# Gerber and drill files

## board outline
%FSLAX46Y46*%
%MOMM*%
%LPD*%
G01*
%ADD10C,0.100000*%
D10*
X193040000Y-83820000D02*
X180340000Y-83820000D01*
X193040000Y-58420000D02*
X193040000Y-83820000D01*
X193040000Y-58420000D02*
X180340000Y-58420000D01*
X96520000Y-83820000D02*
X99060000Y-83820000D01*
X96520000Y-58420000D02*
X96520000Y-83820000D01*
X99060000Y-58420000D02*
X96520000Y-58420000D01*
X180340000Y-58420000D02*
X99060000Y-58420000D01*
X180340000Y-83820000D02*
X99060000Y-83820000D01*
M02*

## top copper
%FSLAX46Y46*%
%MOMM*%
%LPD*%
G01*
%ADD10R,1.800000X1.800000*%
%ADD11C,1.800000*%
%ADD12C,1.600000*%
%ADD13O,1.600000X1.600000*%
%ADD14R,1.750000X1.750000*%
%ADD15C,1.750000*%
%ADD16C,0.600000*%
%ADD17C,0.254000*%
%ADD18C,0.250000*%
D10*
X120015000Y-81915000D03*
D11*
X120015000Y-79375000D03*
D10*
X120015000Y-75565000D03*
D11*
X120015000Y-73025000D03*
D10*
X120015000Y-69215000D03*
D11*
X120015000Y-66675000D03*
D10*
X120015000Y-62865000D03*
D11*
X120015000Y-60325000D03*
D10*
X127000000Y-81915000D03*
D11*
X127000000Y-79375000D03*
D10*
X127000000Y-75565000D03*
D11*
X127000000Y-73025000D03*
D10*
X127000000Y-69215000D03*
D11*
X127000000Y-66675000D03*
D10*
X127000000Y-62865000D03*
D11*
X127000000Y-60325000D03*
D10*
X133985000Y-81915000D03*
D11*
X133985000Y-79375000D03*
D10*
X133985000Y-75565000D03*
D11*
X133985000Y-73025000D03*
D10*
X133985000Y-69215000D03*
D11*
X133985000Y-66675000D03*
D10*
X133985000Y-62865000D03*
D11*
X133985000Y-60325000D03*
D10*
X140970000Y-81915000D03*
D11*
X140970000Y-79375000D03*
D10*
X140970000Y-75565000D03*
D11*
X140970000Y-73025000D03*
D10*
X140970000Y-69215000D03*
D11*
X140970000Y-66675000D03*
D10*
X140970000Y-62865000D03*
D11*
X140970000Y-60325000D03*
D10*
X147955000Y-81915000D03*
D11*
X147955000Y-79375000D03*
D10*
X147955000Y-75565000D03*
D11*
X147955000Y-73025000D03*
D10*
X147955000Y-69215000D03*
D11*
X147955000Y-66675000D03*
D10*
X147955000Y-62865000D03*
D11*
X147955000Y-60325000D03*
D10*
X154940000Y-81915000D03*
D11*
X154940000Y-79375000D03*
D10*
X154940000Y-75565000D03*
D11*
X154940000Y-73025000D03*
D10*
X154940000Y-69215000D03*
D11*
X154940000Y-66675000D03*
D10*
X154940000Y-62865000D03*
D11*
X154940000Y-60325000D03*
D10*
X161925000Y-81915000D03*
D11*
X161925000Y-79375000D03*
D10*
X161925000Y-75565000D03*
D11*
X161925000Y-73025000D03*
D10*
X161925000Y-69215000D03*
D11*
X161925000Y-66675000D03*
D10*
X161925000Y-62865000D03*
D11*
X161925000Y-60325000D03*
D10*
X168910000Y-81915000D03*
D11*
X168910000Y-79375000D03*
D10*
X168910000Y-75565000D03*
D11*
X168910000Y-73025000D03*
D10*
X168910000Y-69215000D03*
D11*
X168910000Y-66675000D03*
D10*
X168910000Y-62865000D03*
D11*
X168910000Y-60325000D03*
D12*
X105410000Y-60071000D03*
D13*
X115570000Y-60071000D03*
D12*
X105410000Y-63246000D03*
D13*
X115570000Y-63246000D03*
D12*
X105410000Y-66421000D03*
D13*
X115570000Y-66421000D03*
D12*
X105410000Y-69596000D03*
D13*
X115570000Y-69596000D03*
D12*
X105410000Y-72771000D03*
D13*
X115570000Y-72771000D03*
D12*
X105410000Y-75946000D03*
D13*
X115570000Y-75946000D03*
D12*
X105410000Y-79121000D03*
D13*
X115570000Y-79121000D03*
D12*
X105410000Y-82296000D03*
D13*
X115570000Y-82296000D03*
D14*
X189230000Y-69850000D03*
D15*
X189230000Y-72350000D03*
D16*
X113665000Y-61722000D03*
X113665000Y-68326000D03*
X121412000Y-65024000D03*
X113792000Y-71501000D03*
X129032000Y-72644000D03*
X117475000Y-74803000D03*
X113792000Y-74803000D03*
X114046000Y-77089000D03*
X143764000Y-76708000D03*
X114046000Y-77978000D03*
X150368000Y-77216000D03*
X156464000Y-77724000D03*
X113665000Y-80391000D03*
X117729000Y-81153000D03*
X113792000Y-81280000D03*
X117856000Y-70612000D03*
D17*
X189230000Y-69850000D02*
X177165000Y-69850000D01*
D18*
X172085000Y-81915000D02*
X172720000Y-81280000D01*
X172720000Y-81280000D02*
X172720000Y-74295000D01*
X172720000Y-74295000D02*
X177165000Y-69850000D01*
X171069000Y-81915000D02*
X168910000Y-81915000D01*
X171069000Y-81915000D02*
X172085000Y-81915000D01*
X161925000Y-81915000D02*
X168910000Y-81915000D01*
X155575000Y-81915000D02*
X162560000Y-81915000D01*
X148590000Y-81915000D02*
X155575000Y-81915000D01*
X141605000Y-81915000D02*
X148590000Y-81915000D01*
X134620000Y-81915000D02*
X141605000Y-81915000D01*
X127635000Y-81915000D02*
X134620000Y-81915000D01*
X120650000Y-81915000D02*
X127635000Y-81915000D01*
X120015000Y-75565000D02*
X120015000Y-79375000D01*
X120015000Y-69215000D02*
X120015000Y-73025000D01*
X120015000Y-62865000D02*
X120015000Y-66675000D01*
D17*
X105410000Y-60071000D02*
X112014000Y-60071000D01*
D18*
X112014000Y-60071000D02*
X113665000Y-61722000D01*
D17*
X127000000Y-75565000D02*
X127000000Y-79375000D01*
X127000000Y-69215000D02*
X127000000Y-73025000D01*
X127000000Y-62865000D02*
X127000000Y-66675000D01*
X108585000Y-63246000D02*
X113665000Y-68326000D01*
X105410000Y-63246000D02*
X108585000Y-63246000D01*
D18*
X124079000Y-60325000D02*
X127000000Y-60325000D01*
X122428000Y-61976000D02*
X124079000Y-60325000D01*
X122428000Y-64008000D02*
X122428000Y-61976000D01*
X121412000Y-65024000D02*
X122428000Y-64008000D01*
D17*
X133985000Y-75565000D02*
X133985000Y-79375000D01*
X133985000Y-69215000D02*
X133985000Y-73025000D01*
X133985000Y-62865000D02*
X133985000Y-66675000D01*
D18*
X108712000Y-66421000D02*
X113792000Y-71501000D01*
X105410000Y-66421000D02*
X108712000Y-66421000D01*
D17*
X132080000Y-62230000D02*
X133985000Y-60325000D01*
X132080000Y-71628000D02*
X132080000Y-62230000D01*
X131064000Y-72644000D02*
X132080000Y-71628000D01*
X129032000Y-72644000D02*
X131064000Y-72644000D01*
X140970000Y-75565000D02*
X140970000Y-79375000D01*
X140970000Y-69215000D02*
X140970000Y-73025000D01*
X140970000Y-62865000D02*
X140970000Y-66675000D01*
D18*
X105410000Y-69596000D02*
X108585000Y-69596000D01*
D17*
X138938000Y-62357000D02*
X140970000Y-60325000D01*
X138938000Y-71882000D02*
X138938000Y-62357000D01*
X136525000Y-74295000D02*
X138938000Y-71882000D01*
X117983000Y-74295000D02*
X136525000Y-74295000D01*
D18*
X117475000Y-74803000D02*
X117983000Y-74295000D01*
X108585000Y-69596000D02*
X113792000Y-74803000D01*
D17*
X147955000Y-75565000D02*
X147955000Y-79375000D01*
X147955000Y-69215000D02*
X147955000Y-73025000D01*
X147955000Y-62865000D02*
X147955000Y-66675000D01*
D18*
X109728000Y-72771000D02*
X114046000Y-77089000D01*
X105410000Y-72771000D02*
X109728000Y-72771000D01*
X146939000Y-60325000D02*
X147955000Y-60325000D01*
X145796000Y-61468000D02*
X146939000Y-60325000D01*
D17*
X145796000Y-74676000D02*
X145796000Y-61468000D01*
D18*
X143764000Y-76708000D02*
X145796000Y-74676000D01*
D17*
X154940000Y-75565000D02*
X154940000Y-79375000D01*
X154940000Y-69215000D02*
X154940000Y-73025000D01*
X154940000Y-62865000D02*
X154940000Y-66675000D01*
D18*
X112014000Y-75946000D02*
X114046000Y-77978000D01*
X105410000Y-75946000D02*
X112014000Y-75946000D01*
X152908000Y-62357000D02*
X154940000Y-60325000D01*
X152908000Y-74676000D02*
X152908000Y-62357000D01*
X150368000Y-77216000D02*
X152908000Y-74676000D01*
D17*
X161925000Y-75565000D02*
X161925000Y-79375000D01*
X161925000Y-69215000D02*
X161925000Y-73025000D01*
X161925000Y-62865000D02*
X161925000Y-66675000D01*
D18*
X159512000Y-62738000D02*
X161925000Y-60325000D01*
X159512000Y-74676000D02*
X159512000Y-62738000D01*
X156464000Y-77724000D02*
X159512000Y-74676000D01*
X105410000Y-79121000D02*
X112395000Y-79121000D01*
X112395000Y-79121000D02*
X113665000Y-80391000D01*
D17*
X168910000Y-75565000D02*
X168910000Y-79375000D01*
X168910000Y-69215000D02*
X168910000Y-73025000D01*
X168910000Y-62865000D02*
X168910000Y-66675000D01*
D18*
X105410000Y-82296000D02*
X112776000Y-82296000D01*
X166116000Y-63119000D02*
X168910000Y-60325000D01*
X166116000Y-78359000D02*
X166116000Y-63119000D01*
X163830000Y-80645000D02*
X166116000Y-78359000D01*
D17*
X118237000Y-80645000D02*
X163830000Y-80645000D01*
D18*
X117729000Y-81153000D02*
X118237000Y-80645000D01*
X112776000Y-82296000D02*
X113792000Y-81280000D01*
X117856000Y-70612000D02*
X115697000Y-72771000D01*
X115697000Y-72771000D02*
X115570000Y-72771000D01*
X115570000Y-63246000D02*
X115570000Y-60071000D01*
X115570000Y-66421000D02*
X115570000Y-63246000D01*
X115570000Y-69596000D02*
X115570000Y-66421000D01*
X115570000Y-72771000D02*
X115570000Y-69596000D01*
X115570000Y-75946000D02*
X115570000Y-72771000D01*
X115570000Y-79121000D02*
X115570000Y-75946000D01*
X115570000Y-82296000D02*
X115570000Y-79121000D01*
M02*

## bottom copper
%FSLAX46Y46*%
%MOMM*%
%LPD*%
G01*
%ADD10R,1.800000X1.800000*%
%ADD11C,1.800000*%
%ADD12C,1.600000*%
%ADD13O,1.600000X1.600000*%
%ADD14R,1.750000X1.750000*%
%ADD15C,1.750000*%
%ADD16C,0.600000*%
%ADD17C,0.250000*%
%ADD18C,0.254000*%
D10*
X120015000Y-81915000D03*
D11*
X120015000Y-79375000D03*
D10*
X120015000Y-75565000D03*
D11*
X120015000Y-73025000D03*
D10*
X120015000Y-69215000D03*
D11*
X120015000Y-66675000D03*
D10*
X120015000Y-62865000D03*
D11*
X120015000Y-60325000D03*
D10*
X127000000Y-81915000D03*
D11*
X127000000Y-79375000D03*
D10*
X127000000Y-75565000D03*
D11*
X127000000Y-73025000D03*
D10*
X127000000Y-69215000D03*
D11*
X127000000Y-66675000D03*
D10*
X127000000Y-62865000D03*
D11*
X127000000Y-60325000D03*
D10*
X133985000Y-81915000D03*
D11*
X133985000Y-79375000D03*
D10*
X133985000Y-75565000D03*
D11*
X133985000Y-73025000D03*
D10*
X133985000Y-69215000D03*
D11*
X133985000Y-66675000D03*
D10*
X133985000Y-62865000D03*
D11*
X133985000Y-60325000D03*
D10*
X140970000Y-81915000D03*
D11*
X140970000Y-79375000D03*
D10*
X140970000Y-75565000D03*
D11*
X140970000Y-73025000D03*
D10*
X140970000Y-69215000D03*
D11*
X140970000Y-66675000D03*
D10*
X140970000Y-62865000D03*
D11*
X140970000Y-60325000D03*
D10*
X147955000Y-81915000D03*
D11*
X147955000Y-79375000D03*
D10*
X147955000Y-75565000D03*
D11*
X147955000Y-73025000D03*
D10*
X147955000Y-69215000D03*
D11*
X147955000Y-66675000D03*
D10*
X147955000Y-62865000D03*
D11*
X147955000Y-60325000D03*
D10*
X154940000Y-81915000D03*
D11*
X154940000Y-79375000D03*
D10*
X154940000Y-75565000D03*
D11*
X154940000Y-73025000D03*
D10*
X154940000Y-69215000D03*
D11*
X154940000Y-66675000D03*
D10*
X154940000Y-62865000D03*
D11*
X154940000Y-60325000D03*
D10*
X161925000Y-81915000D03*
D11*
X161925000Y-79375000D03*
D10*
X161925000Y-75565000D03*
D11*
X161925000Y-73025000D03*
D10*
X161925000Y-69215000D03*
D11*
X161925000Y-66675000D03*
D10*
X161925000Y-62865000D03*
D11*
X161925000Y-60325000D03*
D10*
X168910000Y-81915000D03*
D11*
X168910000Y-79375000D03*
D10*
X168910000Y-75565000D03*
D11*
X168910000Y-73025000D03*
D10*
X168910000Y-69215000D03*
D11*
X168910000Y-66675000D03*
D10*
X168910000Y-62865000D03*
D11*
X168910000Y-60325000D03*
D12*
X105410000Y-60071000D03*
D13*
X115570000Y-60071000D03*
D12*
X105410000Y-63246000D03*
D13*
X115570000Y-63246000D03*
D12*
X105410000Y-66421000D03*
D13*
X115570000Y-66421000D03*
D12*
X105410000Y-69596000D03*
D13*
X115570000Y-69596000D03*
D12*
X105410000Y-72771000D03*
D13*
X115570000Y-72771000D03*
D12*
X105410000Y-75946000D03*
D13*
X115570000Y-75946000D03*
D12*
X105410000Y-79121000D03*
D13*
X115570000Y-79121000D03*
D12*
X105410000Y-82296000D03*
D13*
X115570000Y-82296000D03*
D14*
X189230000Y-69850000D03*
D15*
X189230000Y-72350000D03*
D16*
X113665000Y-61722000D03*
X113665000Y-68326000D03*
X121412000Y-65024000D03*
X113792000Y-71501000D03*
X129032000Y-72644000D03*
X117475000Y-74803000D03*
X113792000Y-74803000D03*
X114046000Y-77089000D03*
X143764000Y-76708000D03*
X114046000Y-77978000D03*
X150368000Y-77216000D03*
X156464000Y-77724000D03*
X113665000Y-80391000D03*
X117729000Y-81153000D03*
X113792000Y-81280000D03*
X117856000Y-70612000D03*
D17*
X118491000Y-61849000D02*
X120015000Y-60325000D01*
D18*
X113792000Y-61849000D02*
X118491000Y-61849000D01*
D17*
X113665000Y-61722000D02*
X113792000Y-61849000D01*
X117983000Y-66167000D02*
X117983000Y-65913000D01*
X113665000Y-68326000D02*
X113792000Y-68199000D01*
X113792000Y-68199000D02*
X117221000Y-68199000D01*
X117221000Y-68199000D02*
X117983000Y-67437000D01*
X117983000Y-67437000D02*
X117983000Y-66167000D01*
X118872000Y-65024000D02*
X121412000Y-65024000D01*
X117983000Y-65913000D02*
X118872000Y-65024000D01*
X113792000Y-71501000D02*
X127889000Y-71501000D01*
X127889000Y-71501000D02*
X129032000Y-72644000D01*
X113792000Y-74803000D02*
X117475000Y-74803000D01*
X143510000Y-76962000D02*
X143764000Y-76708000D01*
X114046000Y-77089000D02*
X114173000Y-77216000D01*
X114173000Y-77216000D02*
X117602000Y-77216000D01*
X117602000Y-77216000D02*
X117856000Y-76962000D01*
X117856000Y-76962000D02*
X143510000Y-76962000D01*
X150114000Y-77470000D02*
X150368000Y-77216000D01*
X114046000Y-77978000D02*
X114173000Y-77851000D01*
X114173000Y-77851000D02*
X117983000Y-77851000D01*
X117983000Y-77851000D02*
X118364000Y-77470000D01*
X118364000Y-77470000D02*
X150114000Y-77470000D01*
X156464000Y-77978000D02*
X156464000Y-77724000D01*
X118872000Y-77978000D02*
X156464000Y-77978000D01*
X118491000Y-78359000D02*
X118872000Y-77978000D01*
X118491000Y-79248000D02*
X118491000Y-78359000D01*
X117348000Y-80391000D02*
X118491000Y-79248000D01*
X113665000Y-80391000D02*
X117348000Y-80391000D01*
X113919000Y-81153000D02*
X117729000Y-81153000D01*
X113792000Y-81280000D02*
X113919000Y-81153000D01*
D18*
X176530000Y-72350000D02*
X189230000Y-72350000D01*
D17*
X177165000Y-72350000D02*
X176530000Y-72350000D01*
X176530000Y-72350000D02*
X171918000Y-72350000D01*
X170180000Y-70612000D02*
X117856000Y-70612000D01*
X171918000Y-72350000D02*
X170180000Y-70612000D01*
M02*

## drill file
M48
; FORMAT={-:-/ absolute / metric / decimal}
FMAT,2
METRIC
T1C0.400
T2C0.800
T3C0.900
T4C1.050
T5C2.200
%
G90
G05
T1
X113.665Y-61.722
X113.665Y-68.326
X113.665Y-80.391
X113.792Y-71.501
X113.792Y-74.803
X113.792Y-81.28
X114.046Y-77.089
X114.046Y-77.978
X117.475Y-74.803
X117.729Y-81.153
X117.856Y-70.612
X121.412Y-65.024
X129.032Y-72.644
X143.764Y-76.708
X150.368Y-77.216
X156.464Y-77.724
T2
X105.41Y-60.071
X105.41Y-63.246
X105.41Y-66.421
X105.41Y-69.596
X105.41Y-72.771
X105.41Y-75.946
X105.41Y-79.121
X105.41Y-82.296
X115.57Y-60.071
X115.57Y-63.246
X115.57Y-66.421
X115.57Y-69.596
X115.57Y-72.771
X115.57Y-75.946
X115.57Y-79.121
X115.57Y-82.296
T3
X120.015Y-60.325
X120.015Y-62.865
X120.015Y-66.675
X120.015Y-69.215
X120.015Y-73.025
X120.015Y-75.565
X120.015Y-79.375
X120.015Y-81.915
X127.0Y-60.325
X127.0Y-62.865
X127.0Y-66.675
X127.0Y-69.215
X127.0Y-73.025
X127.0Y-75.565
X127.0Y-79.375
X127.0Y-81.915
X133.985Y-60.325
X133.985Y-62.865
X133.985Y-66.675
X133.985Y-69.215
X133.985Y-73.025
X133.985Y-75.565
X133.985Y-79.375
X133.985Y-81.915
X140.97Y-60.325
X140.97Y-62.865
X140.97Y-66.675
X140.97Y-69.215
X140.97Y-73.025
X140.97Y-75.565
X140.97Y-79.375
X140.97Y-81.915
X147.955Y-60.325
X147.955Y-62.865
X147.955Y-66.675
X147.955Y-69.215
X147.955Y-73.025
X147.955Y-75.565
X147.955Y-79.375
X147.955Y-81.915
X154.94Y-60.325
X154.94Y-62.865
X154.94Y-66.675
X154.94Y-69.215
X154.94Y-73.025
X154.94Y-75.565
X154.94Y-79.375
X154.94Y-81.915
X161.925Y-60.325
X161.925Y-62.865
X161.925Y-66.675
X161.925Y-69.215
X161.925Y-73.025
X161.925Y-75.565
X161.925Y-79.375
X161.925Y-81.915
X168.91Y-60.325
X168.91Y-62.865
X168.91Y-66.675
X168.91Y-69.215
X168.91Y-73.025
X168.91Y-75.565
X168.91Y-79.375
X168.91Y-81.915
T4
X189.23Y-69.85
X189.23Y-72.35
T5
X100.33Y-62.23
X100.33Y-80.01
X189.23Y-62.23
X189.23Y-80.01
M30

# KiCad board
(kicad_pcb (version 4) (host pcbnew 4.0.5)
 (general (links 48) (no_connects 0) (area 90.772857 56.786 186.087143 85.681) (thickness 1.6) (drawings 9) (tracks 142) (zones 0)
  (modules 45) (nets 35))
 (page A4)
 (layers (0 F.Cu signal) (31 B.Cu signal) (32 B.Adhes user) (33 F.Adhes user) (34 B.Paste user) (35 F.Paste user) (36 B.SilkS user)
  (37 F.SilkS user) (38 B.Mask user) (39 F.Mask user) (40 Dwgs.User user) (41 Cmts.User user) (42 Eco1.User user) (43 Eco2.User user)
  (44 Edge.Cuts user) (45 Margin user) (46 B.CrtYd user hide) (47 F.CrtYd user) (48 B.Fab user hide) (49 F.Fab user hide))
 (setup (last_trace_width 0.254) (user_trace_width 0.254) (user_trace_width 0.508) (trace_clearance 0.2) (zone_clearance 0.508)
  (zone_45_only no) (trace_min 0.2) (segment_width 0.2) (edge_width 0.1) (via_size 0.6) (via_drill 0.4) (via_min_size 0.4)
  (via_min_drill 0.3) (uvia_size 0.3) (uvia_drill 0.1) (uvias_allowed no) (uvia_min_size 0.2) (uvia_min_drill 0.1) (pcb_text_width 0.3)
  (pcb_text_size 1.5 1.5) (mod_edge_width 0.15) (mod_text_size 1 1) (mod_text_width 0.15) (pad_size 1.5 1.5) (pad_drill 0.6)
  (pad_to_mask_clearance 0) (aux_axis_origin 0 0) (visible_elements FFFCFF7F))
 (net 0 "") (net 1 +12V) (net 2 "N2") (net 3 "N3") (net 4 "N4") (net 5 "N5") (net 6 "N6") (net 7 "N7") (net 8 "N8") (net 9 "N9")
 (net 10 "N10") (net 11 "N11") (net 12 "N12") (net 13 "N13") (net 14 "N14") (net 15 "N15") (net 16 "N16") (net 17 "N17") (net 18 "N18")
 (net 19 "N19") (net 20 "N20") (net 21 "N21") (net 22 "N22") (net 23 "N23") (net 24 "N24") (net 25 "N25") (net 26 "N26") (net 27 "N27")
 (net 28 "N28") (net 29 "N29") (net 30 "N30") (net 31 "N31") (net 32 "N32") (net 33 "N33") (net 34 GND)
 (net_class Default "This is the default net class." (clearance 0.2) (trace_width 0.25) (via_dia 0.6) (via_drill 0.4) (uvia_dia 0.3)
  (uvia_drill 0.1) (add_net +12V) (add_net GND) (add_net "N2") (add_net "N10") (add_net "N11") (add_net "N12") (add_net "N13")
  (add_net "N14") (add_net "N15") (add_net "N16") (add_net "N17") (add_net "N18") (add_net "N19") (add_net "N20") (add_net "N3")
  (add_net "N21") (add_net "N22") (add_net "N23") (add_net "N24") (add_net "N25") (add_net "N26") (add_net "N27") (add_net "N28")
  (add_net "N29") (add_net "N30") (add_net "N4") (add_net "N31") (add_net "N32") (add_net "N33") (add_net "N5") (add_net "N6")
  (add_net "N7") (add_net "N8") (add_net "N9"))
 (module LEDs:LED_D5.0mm (layer F.Cu) (at 120.015 81.915 90)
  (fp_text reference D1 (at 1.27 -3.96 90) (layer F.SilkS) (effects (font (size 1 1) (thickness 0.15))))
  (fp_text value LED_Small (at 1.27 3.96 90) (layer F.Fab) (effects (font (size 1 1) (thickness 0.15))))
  (pad 1 thru_hole rect (at 0 0 90) (size 1.8 1.8) (drill 0.9) (layers *.Cu *.Mask) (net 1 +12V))
  (pad 2 thru_hole circle (at 2.54 0 90) (size 1.8 1.8) (drill 0.9) (layers *.Cu *.Mask) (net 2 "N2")))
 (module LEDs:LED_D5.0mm (layer F.Cu) (at 120.015 75.565 90)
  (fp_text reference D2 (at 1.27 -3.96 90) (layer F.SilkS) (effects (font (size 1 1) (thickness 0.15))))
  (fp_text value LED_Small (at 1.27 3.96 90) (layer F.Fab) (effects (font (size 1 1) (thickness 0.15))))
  (pad 1 thru_hole rect (at 0 0 90) (size 1.8 1.8) (drill 0.9) (layers *.Cu *.Mask) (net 2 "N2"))
  (pad 2 thru_hole circle (at 2.54 0 90) (size 1.8 1.8) (drill 0.9) (layers *.Cu *.Mask) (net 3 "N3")))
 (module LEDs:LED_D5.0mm (layer F.Cu) (at 120.015 69.215 90)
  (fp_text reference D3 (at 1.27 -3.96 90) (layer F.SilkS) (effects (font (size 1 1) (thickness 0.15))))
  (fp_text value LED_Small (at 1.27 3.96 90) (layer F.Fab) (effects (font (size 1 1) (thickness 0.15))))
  (pad 1 thru_hole rect (at 0 0 90) (size 1.8 1.8) (drill 0.9) (layers *.Cu *.Mask) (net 3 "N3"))
  (pad 2 thru_hole circle (at 2.54 0 90) (size 1.8 1.8) (drill 0.9) (layers *.Cu *.Mask) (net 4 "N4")))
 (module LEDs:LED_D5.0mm (layer F.Cu) (at 120.015 62.865 90)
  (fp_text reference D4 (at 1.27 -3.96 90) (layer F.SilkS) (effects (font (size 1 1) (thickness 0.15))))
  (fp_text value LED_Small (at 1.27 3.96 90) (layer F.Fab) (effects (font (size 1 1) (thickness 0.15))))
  (pad 1 thru_hole rect (at 0 0 90) (size 1.8 1.8) (drill 0.9) (layers *.Cu *.Mask) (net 4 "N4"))
  (pad 2 thru_hole circle (at 2.54 0 90) (size 1.8 1.8) (drill 0.9) (layers *.Cu *.Mask) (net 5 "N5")))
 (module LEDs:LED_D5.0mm (layer F.Cu) (at 127 81.915 90)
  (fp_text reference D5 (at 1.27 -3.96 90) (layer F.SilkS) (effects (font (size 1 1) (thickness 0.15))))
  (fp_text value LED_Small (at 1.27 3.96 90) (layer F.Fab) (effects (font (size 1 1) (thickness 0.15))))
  (pad 1 thru_hole rect (at 0 0 90) (size 1.8 1.8) (drill 0.9) (layers *.Cu *.Mask) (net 1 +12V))
  (pad 2 thru_hole circle (at 2.54 0 90) (size 1.8 1.8) (drill 0.9) (layers *.Cu *.Mask) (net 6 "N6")))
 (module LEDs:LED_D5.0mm (layer F.Cu) (at 127 75.565 90)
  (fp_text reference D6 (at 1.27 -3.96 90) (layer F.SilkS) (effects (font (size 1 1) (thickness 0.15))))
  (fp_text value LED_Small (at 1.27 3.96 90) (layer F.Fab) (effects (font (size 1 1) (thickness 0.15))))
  (pad 1 thru_hole rect (at 0 0 90) (size 1.8 1.8) (drill 0.9) (layers *.Cu *.Mask) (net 6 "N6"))
  (pad 2 thru_hole circle (at 2.54 0 90) (size 1.8 1.8) (drill 0.9) (layers *.Cu *.Mask) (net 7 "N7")))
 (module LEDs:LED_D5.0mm (layer F.Cu) (at 127 69.215 90)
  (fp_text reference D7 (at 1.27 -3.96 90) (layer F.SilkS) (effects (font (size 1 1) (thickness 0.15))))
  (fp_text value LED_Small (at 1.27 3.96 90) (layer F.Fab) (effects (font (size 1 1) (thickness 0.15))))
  (pad 1 thru_hole rect (at 0 0 90) (size 1.8 1.8) (drill 0.9) (layers *.Cu *.Mask) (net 7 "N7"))
  (pad 2 thru_hole circle (at 2.54 0 90) (size 1.8 1.8) (drill 0.9) (layers *.Cu *.Mask) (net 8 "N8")))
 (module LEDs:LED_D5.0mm (layer F.Cu) (at 127 62.865 90)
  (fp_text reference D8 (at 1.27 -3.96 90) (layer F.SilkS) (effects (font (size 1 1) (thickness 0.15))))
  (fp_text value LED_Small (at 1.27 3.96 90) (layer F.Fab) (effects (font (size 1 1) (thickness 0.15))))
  (pad 1 thru_hole rect (at 0 0 90) (size 1.8 1.8) (drill 0.9) (layers *.Cu *.Mask) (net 8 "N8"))
  (pad 2 thru_hole circle (at 2.54 0 90) (size 1.8 1.8) (drill 0.9) (layers *.Cu *.Mask) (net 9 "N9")))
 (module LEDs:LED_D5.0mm (layer F.Cu) (at 133.985 81.915 90)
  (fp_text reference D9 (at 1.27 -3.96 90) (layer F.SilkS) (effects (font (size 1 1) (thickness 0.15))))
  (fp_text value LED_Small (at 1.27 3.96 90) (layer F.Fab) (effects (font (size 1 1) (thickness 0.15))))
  (pad 1 thru_hole rect (at 0 0 90) (size 1.8 1.8) (drill 0.9) (layers *.Cu *.Mask) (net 1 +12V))
  (pad 2 thru_hole circle (at 2.54 0 90) (size 1.8 1.8) (drill 0.9) (layers *.Cu *.Mask) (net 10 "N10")))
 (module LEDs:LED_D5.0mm (layer F.Cu) (at 133.985 75.565 90)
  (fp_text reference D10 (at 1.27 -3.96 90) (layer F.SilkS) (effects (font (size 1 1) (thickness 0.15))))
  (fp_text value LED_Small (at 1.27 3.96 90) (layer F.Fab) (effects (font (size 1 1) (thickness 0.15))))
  (pad 1 thru_hole rect (at 0 0 90) (size 1.8 1.8) (drill 0.9) (layers *.Cu *.Mask) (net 10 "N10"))
  (pad 2 thru_hole circle (at 2.54 0 90) (size 1.8 1.8) (drill 0.9) (layers *.Cu *.Mask) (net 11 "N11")))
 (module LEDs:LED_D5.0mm (layer F.Cu) (at 133.985 69.215 90)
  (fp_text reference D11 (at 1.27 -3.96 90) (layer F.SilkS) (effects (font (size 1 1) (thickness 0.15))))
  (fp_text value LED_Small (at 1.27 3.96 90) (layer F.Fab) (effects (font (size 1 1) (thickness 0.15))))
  (pad 1 thru_hole rect (at 0 0 90) (size 1.8 1.8) (drill 0.9) (layers *.Cu *.Mask) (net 11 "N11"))
  (pad 2 thru_hole circle (at 2.54 0 90) (size 1.8 1.8) (drill 0.9) (layers *.Cu *.Mask) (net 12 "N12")))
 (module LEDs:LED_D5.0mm (layer F.Cu) (at 133.985 62.865 90)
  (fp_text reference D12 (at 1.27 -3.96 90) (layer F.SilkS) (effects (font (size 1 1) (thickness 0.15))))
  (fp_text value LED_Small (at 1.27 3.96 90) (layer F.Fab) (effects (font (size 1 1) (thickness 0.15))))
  (pad 1 thru_hole rect (at 0 0 90) (size 1.8 1.8) (drill 0.9) (layers *.Cu *.Mask) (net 12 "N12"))
  (pad 2 thru_hole circle (at 2.54 0 90) (size 1.8 1.8) (drill 0.9) (layers *.Cu *.Mask) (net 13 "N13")))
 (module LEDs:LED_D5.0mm (layer F.Cu) (at 140.97 81.915 90)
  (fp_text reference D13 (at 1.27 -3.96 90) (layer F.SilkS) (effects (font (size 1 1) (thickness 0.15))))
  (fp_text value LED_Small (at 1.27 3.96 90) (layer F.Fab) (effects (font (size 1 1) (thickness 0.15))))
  (pad 1 thru_hole rect (at 0 0 90) (size 1.8 1.8) (drill 0.9) (layers *.Cu *.Mask) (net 1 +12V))
  (pad 2 thru_hole circle (at 2.54 0 90) (size 1.8 1.8) (drill 0.9) (layers *.Cu *.Mask) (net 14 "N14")))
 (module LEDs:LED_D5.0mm (layer F.Cu) (at 140.97 75.565 90)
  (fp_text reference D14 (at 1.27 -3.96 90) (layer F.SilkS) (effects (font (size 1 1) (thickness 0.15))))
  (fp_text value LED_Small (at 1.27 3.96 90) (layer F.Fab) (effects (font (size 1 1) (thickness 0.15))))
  (pad 1 thru_hole rect (at 0 0 90) (size 1.8 1.8) (drill 0.9) (layers *.Cu *.Mask) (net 14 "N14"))
  (pad 2 thru_hole circle (at 2.54 0 90) (size 1.8 1.8) (drill 0.9) (layers *.Cu *.Mask) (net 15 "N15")))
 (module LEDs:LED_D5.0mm (layer F.Cu) (at 140.97 69.215 90)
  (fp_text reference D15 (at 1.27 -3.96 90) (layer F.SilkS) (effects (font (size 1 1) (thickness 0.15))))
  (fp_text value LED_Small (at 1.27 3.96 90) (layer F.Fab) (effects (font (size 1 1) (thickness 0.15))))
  (pad 1 thru_hole rect (at 0 0 90) (size 1.8 1.8) (drill 0.9) (layers *.Cu *.Mask) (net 15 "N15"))
  (pad 2 thru_hole circle (at 2.54 0 90) (size 1.8 1.8) (drill 0.9) (layers *.Cu *.Mask) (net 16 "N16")))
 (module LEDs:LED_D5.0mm (layer F.Cu) (at 140.97 62.865 90)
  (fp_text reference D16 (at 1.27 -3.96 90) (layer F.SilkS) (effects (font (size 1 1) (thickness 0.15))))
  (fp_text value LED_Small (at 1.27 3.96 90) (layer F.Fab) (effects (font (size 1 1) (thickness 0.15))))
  (pad 1 thru_hole rect (at 0 0 90) (size 1.8 1.8) (drill 0.9) (layers *.Cu *.Mask) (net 16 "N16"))
  (pad 2 thru_hole circle (at 2.54 0 90) (size 1.8 1.8) (drill 0.9) (layers *.Cu *.Mask) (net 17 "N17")))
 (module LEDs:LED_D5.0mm (layer F.Cu) (at 147.955 81.915 90)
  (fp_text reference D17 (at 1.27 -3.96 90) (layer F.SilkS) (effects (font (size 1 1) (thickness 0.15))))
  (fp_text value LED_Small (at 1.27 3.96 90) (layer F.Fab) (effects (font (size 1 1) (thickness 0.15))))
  (pad 1 thru_hole rect (at 0 0 90) (size 1.8 1.8) (drill 0.9) (layers *.Cu *.Mask) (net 1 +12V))
  (pad 2 thru_hole circle (at 2.54 0 90) (size 1.8 1.8) (drill 0.9) (layers *.Cu *.Mask) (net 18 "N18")))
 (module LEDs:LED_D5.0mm (layer F.Cu) (at 147.955 75.565 90)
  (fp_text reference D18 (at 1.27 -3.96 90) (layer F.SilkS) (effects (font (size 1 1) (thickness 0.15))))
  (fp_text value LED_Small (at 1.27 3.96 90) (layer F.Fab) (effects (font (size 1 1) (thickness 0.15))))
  (pad 1 thru_hole rect (at 0 0 90) (size 1.8 1.8) (drill 0.9) (layers *.Cu *.Mask) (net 18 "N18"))
  (pad 2 thru_hole circle (at 2.54 0 90) (size 1.8 1.8) (drill 0.9) (layers *.Cu *.Mask) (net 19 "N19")))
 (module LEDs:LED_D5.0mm (layer F.Cu) (at 147.955 69.215 90)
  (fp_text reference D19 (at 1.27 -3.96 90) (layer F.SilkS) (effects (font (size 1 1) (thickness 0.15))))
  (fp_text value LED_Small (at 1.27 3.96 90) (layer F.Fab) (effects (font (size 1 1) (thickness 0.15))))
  (pad 1 thru_hole rect (at 0 0 90) (size 1.8 1.8) (drill 0.9) (layers *.Cu *.Mask) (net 19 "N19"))
  (pad 2 thru_hole circle (at 2.54 0 90) (size 1.8 1.8) (drill 0.9) (layers *.Cu *.Mask) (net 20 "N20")))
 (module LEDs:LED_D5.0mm (layer F.Cu) (at 147.955 62.865 90)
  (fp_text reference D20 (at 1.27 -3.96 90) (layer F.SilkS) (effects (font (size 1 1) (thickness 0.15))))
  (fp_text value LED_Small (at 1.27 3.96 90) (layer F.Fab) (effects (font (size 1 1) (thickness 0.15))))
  (pad 1 thru_hole rect (at 0 0 90) (size 1.8 1.8) (drill 0.9) (layers *.Cu *.Mask) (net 20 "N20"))
  (pad 2 thru_hole circle (at 2.54 0 90) (size 1.8 1.8) (drill 0.9) (layers *.Cu *.Mask) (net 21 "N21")))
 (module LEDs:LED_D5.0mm (layer F.Cu) (at 154.94 81.915 90)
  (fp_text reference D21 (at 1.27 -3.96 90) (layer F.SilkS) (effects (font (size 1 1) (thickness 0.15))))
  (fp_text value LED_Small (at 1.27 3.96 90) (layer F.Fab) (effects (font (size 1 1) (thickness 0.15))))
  (pad 1 thru_hole rect (at 0 0 90) (size 1.8 1.8) (drill 0.9) (layers *.Cu *.Mask) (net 1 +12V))
  (pad 2 thru_hole circle (at 2.54 0 90) (size 1.8 1.8) (drill 0.9) (layers *.Cu *.Mask) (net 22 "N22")))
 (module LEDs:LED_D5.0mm (layer F.Cu) (at 154.94 75.565 90)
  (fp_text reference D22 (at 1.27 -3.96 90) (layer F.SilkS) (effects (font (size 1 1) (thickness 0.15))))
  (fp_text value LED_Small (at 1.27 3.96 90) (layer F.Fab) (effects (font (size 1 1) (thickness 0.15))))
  (pad 1 thru_hole rect (at 0 0 90) (size 1.8 1.8) (drill 0.9) (layers *.Cu *.Mask) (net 22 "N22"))
  (pad 2 thru_hole circle (at 2.54 0 90) (size 1.8 1.8) (drill 0.9) (layers *.Cu *.Mask) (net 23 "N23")))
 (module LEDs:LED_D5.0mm (layer F.Cu) (at 154.94 69.215 90)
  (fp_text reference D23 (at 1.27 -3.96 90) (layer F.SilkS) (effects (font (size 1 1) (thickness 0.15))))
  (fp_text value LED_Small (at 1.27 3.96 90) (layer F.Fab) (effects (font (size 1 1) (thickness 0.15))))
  (pad 1 thru_hole rect (at 0 0 90) (size 1.8 1.8) (drill 0.9) (layers *.Cu *.Mask) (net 23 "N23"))
  (pad 2 thru_hole circle (at 2.54 0 90) (size 1.8 1.8) (drill 0.9) (layers *.Cu *.Mask) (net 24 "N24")))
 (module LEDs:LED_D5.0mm (layer F.Cu) (at 154.94 62.865 90)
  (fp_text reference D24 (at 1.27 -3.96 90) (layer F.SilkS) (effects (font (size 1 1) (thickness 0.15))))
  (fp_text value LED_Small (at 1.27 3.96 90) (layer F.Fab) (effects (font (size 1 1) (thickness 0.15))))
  (pad 1 thru_hole rect (at 0 0 90) (size 1.8 1.8) (drill 0.9) (layers *.Cu *.Mask) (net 24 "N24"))
  (pad 2 thru_hole circle (at 2.54 0 90) (size 1.8 1.8) (drill 0.9) (layers *.Cu *.Mask) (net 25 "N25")))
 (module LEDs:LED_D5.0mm (layer F.Cu) (at 161.925 81.915 90)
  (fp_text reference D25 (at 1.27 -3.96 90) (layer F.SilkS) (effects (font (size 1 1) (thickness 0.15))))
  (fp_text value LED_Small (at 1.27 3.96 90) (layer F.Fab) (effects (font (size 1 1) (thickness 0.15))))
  (pad 1 thru_hole rect (at 0 0 90) (size 1.8 1.8) (drill 0.9) (layers *.Cu *.Mask) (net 1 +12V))
  (pad 2 thru_hole circle (at 2.54 0 90) (size 1.8 1.8) (drill 0.9) (layers *.Cu *.Mask) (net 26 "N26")))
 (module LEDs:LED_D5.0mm (layer F.Cu) (at 161.925 75.565 90)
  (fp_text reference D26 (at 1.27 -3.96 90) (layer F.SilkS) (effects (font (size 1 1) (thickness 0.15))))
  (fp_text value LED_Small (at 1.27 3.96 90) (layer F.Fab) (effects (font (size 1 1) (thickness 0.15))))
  (pad 1 thru_hole rect (at 0 0 90) (size 1.8 1.8) (drill 0.9) (layers *.Cu *.Mask) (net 26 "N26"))
  (pad 2 thru_hole circle (at 2.54 0 90) (size 1.8 1.8) (drill 0.9) (layers *.Cu *.Mask) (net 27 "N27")))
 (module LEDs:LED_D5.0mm (layer F.Cu) (at 161.925 69.215 90)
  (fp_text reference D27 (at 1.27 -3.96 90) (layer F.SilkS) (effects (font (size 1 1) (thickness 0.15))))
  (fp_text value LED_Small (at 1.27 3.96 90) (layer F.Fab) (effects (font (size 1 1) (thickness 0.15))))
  (pad 1 thru_hole rect (at 0 0 90) (size 1.8 1.8) (drill 0.9) (layers *.Cu *.Mask) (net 27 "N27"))
  (pad 2 thru_hole circle (at 2.54 0 90) (size 1.8 1.8) (drill 0.9) (layers *.Cu *.Mask) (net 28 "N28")))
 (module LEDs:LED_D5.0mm (layer F.Cu) (at 161.925 62.865 90)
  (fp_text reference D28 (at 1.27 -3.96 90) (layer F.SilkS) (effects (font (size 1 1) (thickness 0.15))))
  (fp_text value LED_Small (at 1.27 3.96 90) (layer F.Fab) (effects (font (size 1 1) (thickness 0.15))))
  (pad 1 thru_hole rect (at 0 0 90) (size 1.8 1.8) (drill 0.9) (layers *.Cu *.Mask) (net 28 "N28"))
  (pad 2 thru_hole circle (at 2.54 0 90) (size 1.8 1.8) (drill 0.9) (layers *.Cu *.Mask) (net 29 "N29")))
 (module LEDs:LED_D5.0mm (layer F.Cu) (at 168.91 81.915 90)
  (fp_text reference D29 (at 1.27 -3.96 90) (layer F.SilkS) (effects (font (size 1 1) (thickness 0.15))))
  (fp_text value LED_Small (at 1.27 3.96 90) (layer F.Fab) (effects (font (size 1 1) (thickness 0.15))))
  (pad 1 thru_hole rect (at 0 0 90) (size 1.8 1.8) (drill 0.9) (layers *.Cu *.Mask) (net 1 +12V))
  (pad 2 thru_hole circle (at 2.54 0 90) (size 1.8 1.8) (drill 0.9) (layers *.Cu *.Mask) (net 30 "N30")))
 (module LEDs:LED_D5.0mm (layer F.Cu) (at 168.91 75.565 90)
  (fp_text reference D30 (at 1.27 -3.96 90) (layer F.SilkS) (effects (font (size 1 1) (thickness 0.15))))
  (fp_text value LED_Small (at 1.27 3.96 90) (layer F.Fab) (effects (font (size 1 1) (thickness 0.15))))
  (pad 1 thru_hole rect (at 0 0 90) (size 1.8 1.8) (drill 0.9) (layers *.Cu *.Mask) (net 30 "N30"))
  (pad 2 thru_hole circle (at 2.54 0 90) (size 1.8 1.8) (drill 0.9) (layers *.Cu *.Mask) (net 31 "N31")))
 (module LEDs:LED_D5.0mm (layer F.Cu) (at 168.91 69.215 90)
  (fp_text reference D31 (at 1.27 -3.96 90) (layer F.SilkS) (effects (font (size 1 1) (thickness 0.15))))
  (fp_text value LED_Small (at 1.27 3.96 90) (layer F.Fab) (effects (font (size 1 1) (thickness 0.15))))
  (pad 1 thru_hole rect (at 0 0 90) (size 1.8 1.8) (drill 0.9) (layers *.Cu *.Mask) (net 31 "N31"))
  (pad 2 thru_hole circle (at 2.54 0 90) (size 1.8 1.8) (drill 0.9) (layers *.Cu *.Mask) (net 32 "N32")))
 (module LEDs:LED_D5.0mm (layer F.Cu) (at 168.91 62.865 90)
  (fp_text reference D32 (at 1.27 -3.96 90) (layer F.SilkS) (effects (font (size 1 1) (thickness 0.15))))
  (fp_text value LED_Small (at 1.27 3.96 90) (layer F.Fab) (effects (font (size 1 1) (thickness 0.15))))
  (pad 1 thru_hole rect (at 0 0 90) (size 1.8 1.8) (drill 0.9) (layers *.Cu *.Mask) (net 32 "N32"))
  (pad 2 thru_hole circle (at 2.54 0 90) (size 1.8 1.8) (drill 0.9) (layers *.Cu *.Mask) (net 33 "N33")))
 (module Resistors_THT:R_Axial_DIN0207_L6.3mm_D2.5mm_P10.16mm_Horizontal (layer F.Cu) (at 105.41 60.071)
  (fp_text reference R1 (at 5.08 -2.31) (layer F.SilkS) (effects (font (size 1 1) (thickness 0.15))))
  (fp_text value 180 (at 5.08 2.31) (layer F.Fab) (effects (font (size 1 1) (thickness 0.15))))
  (pad 1 thru_hole circle (at 0 0) (size 1.6 1.6) (drill 0.8) (layers *.Cu *.Mask) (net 5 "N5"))
  (pad 2 thru_hole oval (at 10.16 0) (size 1.6 1.6) (drill 0.8) (layers *.Cu *.Mask) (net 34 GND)))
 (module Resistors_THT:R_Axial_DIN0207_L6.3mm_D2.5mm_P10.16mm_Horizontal (layer F.Cu) (at 105.41 63.246)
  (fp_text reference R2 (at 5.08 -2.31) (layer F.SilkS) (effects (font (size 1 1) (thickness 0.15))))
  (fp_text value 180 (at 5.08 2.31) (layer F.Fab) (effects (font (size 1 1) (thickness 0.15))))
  (pad 1 thru_hole circle (at 0 0) (size 1.6 1.6) (drill 0.8) (layers *.Cu *.Mask) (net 9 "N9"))
  (pad 2 thru_hole oval (at 10.16 0) (size 1.6 1.6) (drill 0.8) (layers *.Cu *.Mask) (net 34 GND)))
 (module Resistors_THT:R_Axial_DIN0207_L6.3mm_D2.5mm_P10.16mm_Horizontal (layer F.Cu) (at 105.41 66.421)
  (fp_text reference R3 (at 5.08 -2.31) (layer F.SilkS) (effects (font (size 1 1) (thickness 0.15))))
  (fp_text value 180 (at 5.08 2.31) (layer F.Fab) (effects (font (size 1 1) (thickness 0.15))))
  (pad 1 thru_hole circle (at 0 0) (size 1.6 1.6) (drill 0.8) (layers *.Cu *.Mask) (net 13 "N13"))
  (pad 2 thru_hole oval (at 10.16 0) (size 1.6 1.6) (drill 0.8) (layers *.Cu *.Mask) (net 34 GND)))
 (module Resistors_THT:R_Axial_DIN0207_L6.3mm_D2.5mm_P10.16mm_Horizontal (layer F.Cu) (at 105.41 69.596)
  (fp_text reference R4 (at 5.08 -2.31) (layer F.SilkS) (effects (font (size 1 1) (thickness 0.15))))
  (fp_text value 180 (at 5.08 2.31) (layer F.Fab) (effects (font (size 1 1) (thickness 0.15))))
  (pad 1 thru_hole circle (at 0 0) (size 1.6 1.6) (drill 0.8) (layers *.Cu *.Mask) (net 17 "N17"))
  (pad 2 thru_hole oval (at 10.16 0) (size 1.6 1.6) (drill 0.8) (layers *.Cu *.Mask) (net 34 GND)))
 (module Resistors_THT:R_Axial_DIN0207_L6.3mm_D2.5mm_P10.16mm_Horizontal (layer F.Cu) (at 105.41 72.771)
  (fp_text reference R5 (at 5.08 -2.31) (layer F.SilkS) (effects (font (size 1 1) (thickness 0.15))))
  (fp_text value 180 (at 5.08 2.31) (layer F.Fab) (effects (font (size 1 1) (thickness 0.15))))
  (pad 1 thru_hole circle (at 0 0) (size 1.6 1.6) (drill 0.8) (layers *.Cu *.Mask) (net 21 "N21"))
  (pad 2 thru_hole oval (at 10.16 0) (size 1.6 1.6) (drill 0.8) (layers *.Cu *.Mask) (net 34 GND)))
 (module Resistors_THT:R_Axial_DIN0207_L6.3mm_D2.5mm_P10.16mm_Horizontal (layer F.Cu) (at 105.41 75.946)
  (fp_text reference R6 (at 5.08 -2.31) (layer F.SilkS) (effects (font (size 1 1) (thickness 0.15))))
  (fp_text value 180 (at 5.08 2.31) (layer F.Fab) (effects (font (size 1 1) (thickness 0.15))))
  (pad 1 thru_hole circle (at 0 0) (size 1.6 1.6) (drill 0.8) (layers *.Cu *.Mask) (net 25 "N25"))
  (pad 2 thru_hole oval (at 10.16 0) (size 1.6 1.6) (drill 0.8) (layers *.Cu *.Mask) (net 34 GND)))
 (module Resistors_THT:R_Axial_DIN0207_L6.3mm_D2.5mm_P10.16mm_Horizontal (layer F.Cu) (at 105.41 79.121)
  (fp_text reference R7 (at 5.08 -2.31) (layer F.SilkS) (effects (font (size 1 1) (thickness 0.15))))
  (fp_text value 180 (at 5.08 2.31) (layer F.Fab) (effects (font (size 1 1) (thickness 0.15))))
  (pad 1 thru_hole circle (at 0 0) (size 1.6 1.6) (drill 0.8) (layers *.Cu *.Mask) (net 29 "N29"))
  (pad 2 thru_hole oval (at 10.16 0) (size 1.6 1.6) (drill 0.8) (layers *.Cu *.Mask) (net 34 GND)))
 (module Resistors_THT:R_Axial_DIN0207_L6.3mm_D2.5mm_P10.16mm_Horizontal (layer F.Cu) (at 105.41 82.296)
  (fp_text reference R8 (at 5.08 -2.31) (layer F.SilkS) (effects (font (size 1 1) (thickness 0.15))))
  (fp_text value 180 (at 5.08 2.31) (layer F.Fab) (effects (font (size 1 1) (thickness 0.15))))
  (pad 1 thru_hole circle (at 0 0) (size 1.6 1.6) (drill 0.8) (layers *.Cu *.Mask) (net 33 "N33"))
  (pad 2 thru_hole oval (at 10.16 0) (size 1.6 1.6) (drill 0.8) (layers *.Cu *.Mask) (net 34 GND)))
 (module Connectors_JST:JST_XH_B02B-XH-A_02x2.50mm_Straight (layer F.Cu) (at 189.23 69.85 270)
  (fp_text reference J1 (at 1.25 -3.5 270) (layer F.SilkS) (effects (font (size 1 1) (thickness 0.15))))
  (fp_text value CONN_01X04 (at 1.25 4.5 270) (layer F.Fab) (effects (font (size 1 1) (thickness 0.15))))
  (pad 1 thru_hole rect (at 0 0 270) (size 1.75 1.75) (drill 1.05) (layers *.Cu *.Mask) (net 1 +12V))
  (pad 2 thru_hole circle (at 2.5 0 270) (size 1.75 1.75) (drill 1.05) (layers *.Cu *.Mask) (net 34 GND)))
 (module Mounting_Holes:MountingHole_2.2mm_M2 (layer F.Cu) (at 189.23 62.23)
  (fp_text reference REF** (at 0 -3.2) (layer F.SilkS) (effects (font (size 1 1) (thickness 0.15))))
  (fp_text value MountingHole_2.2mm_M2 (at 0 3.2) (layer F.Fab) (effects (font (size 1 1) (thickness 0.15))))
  (pad 1 np_thru_hole circle (at 0 0) (size 2.2 2.2) (drill 2.2) (layers *.Cu *.Mask)))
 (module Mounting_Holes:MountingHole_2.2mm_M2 (layer F.Cu) (at 189.23 80.01)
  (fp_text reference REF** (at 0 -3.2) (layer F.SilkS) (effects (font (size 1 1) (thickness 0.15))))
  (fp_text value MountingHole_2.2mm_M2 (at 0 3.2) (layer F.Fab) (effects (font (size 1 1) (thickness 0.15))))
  (pad 1 np_thru_hole circle (at 0 0) (size 2.2 2.2) (drill 2.2) (layers *.Cu *.Mask)))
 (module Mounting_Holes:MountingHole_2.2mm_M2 (layer F.Cu) (at 100.33 62.23)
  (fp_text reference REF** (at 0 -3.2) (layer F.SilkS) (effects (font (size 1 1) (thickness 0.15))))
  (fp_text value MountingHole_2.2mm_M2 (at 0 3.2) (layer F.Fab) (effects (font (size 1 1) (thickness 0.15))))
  (pad 1 np_thru_hole circle (at 0 0) (size 2.2 2.2) (drill 2.2) (layers *.Cu *.Mask)))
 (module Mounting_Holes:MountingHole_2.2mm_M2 (layer F.Cu) (at 100.33 80.01)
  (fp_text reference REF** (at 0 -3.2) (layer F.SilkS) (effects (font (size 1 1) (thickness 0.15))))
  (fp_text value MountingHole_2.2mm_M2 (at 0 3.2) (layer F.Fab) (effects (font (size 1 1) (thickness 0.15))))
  (pad 1 np_thru_hole circle (at 0 0) (size 2.2 2.2) (drill 2.2) (layers *.Cu *.Mask)))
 (gr_line (start 193.04 83.82) (end 180.34 83.82) (angle 90) (layer Edge.Cuts) (width 0.1))
 (gr_line (start 193.04 58.42) (end 193.04 83.82) (angle 90) (layer Edge.Cuts) (width 0.1))
 (gr_line (start 193.04 58.42) (end 180.34 58.42) (angle 90) (layer Edge.Cuts) (width 0.1))
 (gr_line (start 96.52 83.82) (end 99.06 83.82) (angle 90) (layer Edge.Cuts) (width 0.1))
 (gr_line (start 96.52 58.42) (end 96.52 83.82) (angle 90) (layer Edge.Cuts) (width 0.1))
 (gr_line (start 99.06 58.42) (end 96.52 58.42) (angle 90) (layer Edge.Cuts) (width 0.1))
 (gr_line (start 180.34 58.42) (end 99.06 58.42) (angle 90) (layer Edge.Cuts) (width 0.1))
 (gr_line (start 180.34 83.82) (end 99.06 83.82) (angle 90) (layer Edge.Cuts) (width 0.1))
 (segment (start 189.23 69.85) (end 177.165 69.85) (width 0.254) (layer F.Cu) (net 1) (status 400000))
 (segment (start 172.085 81.915) (end 172.72 81.28) (width 0.25) (layer F.Cu) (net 1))
 (segment (start 172.72 81.28) (end 172.72 74.295) (width 0.25) (layer F.Cu) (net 1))
 (segment (start 172.72 74.295) (end 177.165 69.85) (width 0.25) (layer F.Cu) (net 1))
 (segment (start 171.069 81.915) (end 168.91 81.915) (width 0.25) (layer F.Cu) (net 1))
 (segment (start 171.069 81.915) (end 172.085 81.915) (width 0.25) (layer F.Cu) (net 1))
 (segment (start 161.925 81.915) (end 168.91 81.915) (width 0.25) (layer F.Cu) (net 1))
 (segment (start 155.575 81.915) (end 162.56 81.915) (width 0.25) (layer F.Cu) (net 1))
 (segment (start 148.59 81.915) (end 155.575 81.915) (width 0.25) (layer F.Cu) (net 1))
 (segment (start 141.605 81.915) (end 148.59 81.915) (width 0.25) (layer F.Cu) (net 1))
 (segment (start 134.62 81.915) (end 141.605 81.915) (width 0.25) (layer F.Cu) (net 1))
 (segment (start 127.635 81.915) (end 134.62 81.915) (width 0.25) (layer F.Cu) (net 1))
 (segment (start 120.65 81.915) (end 127.635 81.915) (width 0.25) (layer F.Cu) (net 1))
 (segment (start 120.015 75.565) (end 120.015 79.375) (width 0.25) (layer F.Cu) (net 2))
 (segment (start 120.015 69.215) (end 120.015 73.025) (width 0.25) (layer F.Cu) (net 3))
 (segment (start 120.015 62.865) (end 120.015 66.675) (width 0.25) (layer F.Cu) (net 4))
 (segment (start 105.41 60.071) (end 112.014 60.071) (width 0.254) (layer F.Cu) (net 5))
 (segment (start 118.491 61.849) (end 120.015 60.325) (width 0.25) (layer B.Cu) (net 5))
 (segment (start 113.792 61.849) (end 118.491 61.849) (width 0.254) (layer B.Cu) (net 5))
 (segment (start 113.665 61.722) (end 113.792 61.849) (width 0.25) (layer B.Cu) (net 5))
 (via (at 113.665 61.722) (size 0.6) (drill 0.4) (layers F.Cu B.Cu) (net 5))
 (segment (start 112.014 60.071) (end 113.665 61.722) (width 0.25) (layer F.Cu) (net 5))
 (segment (start 127 75.565) (end 127 79.375) (width 0.254) (layer F.Cu) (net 6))
 (segment (start 127 69.215) (end 127 73.025) (width 0.254) (layer F.Cu) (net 7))
 (segment (start 127 62.865) (end 127 66.675) (width 0.254) (layer F.Cu) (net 8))
 (segment (start 117.983 66.167) (end 117.983 65.913) (width 0.25) (layer B.Cu) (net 9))
 (segment (start 108.585 63.246) (end 113.665 68.326) (width 0.254) (layer F.Cu) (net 9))
 (via (at 113.665 68.326) (size 0.6) (drill 0.4) (layers F.Cu B.Cu) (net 9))
 (segment (start 113.665 68.326) (end 113.792 68.199) (width 0.25) (layer B.Cu) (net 9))
 (segment (start 113.792 68.199) (end 117.221 68.199) (width 0.25) (layer B.Cu) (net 9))
 (segment (start 117.221 68.199) (end 117.983 67.437) (width 0.25) (layer B.Cu) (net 9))
 (segment (start 117.983 67.437) (end 117.983 66.167) (width 0.25) (layer B.Cu) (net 9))
 (segment (start 105.41 63.246) (end 108.585 63.246) (width 0.254) (layer F.Cu) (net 9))
 (segment (start 124.079 60.325) (end 127 60.325) (width 0.25) (layer F.Cu) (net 9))
 (segment (start 122.428 61.976) (end 124.079 60.325) (width 0.25) (layer F.Cu) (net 9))
 (segment (start 122.428 64.008) (end 122.428 61.976) (width 0.25) (layer F.Cu) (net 9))
 (segment (start 121.412 65.024) (end 122.428 64.008) (width 0.25) (layer F.Cu) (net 9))
 (via (at 121.412 65.024) (size 0.6) (drill 0.4) (layers F.Cu B.Cu) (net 9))
 (segment (start 118.872 65.024) (end 121.412 65.024) (width 0.25) (layer B.Cu) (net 9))
 (segment (start 117.983 65.913) (end 118.872 65.024) (width 0.25) (layer B.Cu) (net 9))
 (segment (start 133.985 75.565) (end 133.985 79.375) (width 0.254) (layer F.Cu) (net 10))
 (segment (start 133.985 69.215) (end 133.985 73.025) (width 0.254) (layer F.Cu) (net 11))
 (segment (start 133.985 62.865) (end 133.985 66.675) (width 0.254) (layer F.Cu) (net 12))
 (segment (start 113.792 71.501) (end 127.889 71.501) (width 0.25) (layer B.Cu) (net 13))
 (segment (start 108.712 66.421) (end 113.792 71.501) (width 0.25) (layer F.Cu) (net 13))
 (via (at 113.792 71.501) (size 0.6) (drill 0.4) (layers F.Cu B.Cu) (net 13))
 (segment (start 105.41 66.421) (end 108.712 66.421) (width 0.25) (layer F.Cu) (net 13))
 (segment (start 132.08 62.23) (end 133.985 60.325) (width 0.254) (layer F.Cu) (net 13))
 (segment (start 132.08 71.628) (end 132.08 62.23) (width 0.254) (layer F.Cu) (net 13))
 (segment (start 131.064 72.644) (end 132.08 71.628) (width 0.254) (layer F.Cu) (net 13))
 (segment (start 129.032 72.644) (end 131.064 72.644) (width 0.254) (layer F.Cu) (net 13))
 (via (at 129.032 72.644) (size 0.6) (drill 0.4) (layers F.Cu B.Cu) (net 13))
 (segment (start 127.889 71.501) (end 129.032 72.644) (width 0.25) (layer B.Cu) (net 13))
 (segment (start 140.97 75.565) (end 140.97 79.375) (width 0.254) (layer F.Cu) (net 14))
 (segment (start 140.97 69.215) (end 140.97 73.025) (width 0.254) (layer F.Cu) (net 15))
 (segment (start 140.97 62.865) (end 140.97 66.675) (width 0.254) (layer F.Cu) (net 16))
 (segment (start 105.41 69.596) (end 108.585 69.596) (width 0.25) (layer F.Cu) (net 17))
 (segment (start 138.938 62.357) (end 140.97 60.325) (width 0.254) (layer F.Cu) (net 17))
 (segment (start 138.938 71.882) (end 138.938 62.357) (width 0.254) (layer F.Cu) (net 17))
 (segment (start 136.525 74.295) (end 138.938 71.882) (width 0.254) (layer F.Cu) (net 17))
 (segment (start 117.983 74.295) (end 136.525 74.295) (width 0.254) (layer F.Cu) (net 17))
 (segment (start 117.475 74.803) (end 117.983 74.295) (width 0.25) (layer F.Cu) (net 17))
 (via (at 117.475 74.803) (size 0.6) (drill 0.4) (layers F.Cu B.Cu) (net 17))
 (segment (start 113.792 74.803) (end 117.475 74.803) (width 0.25) (layer B.Cu) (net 17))
 (via (at 113.792 74.803) (size 0.6) (drill 0.4) (layers F.Cu B.Cu) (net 17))
 (segment (start 108.585 69.596) (end 113.792 74.803) (width 0.25) (layer F.Cu) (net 17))
 (segment (start 147.955 75.565) (end 147.955 79.375) (width 0.254) (layer F.Cu) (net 18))
 (segment (start 147.955 69.215) (end 147.955 73.025) (width 0.254) (layer F.Cu) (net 19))
 (segment (start 147.955 62.865) (end 147.955 66.675) (width 0.254) (layer F.Cu) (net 20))
 (segment (start 143.51 76.962) (end 143.764 76.708) (width 0.25) (layer B.Cu) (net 21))
 (segment (start 109.728 72.771) (end 114.046 77.089) (width 0.25) (layer F.Cu) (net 21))
 (via (at 114.046 77.089) (size 0.6) (drill 0.4) (layers F.Cu B.Cu) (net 21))
 (segment (start 114.046 77.089) (end 114.173 77.216) (width 0.25) (layer B.Cu) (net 21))
 (segment (start 114.173 77.216) (end 117.602 77.216) (width 0.25) (layer B.Cu) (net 21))
 (segment (start 117.602 77.216) (end 117.856 76.962) (width 0.25) (layer B.Cu) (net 21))
 (segment (start 117.856 76.962) (end 143.51 76.962) (width 0.25) (layer B.Cu) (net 21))
 (segment (start 105.41 72.771) (end 109.728 72.771) (width 0.25) (layer F.Cu) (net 21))
 (segment (start 146.939 60.325) (end 147.955 60.325) (width 0.25) (layer F.Cu) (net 21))
 (segment (start 145.796 61.468) (end 146.939 60.325) (width 0.25) (layer F.Cu) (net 21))
 (segment (start 145.796 74.676) (end 145.796 61.468) (width 0.254) (layer F.Cu) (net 21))
 (segment (start 143.764 76.708) (end 145.796 74.676) (width 0.25) (layer F.Cu) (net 21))
 (via (at 143.764 76.708) (size 0.6) (drill 0.4) (layers F.Cu B.Cu) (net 21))
 (segment (start 154.94 75.565) (end 154.94 79.375) (width 0.254) (layer F.Cu) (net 22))
 (segment (start 154.94 69.215) (end 154.94 73.025) (width 0.254) (layer F.Cu) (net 23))
 (segment (start 154.94 62.865) (end 154.94 66.675) (width 0.254) (layer F.Cu) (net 24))
 (segment (start 150.114 77.47) (end 150.368 77.216) (width 0.25) (layer B.Cu) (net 25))
 (segment (start 112.014 75.946) (end 114.046 77.978) (width 0.25) (layer F.Cu) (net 25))
 (via (at 114.046 77.978) (size 0.6) (drill 0.4) (layers F.Cu B.Cu) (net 25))
 (segment (start 114.046 77.978) (end 114.173 77.851) (width 0.25) (layer B.Cu) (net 25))
 (segment (start 114.173 77.851) (end 117.983 77.851) (width 0.25) (layer B.Cu) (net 25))
 (segment (start 117.983 77.851) (end 118.364 77.47) (width 0.25) (layer B.Cu) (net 25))
 (segment (start 118.364 77.47) (end 150.114 77.47) (width 0.25) (layer B.Cu) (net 25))
 (segment (start 105.41 75.946) (end 112.014 75.946) (width 0.25) (layer F.Cu) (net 25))
 (segment (start 152.908 62.357) (end 154.94 60.325) (width 0.25) (layer F.Cu) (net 25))
 (segment (start 152.908 74.676) (end 152.908 62.357) (width 0.25) (layer F.Cu) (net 25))
 (segment (start 150.368 77.216) (end 152.908 74.676) (width 0.25) (layer F.Cu) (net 25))
 (via (at 150.368 77.216) (size 0.6) (drill 0.4) (layers F.Cu B.Cu) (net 25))
 (segment (start 161.925 75.565) (end 161.925 79.375) (width 0.254) (layer F.Cu) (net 26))
 (segment (start 161.925 69.215) (end 161.925 73.025) (width 0.254) (layer F.Cu) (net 27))
 (segment (start 161.925 62.865) (end 161.925 66.675) (width 0.254) (layer F.Cu) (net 28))
 (segment (start 156.464 77.978) (end 156.464 77.724) (width 0.25) (layer B.Cu) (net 29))
 (segment (start 159.512 62.738) (end 161.925 60.325) (width 0.25) (layer F.Cu) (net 29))
 (segment (start 159.512 74.676) (end 159.512 62.738) (width 0.25) (layer F.Cu) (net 29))
 (segment (start 156.464 77.724) (end 159.512 74.676) (width 0.25) (layer F.Cu) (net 29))
 (via (at 156.464 77.724) (size 0.6) (drill 0.4) (layers F.Cu B.Cu) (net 29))
 (segment (start 105.41 79.121) (end 112.395 79.121) (width 0.25) (layer F.Cu) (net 29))
 (segment (start 118.872 77.978) (end 156.464 77.978) (width 0.25) (layer B.Cu) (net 29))
 (segment (start 118.491 78.359) (end 118.872 77.978) (width 0.25) (layer B.Cu) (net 29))
 (segment (start 118.491 79.248) (end 118.491 78.359) (width 0.25) (layer B.Cu) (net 29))
 (segment (start 117.348 80.391) (end 118.491 79.248) (width 0.25) (layer B.Cu) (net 29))
 (segment (start 113.665 80.391) (end 117.348 80.391) (width 0.25) (layer B.Cu) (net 29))
 (via (at 113.665 80.391) (size 0.6) (drill 0.4) (layers F.Cu B.Cu) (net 29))
 (segment (start 112.395 79.121) (end 113.665 80.391) (width 0.25) (layer F.Cu) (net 29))
 (segment (start 168.91 75.565) (end 168.91 79.375) (width 0.254) (layer F.Cu) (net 30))
 (segment (start 168.91 69.215) (end 168.91 73.025) (width 0.254) (layer F.Cu) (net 31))
 (segment (start 168.91 62.865) (end 168.91 66.675) (width 0.254) (layer F.Cu) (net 32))
 (segment (start 105.41 82.296) (end 112.776 82.296) (width 0.25) (layer F.Cu) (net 33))
 (segment (start 166.116 63.119) (end 168.91 60.325) (width 0.25) (layer F.Cu) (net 33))
 (segment (start 166.116 78.359) (end 166.116 63.119) (width 0.25) (layer F.Cu) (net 33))
 (segment (start 163.83 80.645) (end 166.116 78.359) (width 0.25) (layer F.Cu) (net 33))
 (segment (start 118.237 80.645) (end 163.83 80.645) (width 0.254) (layer F.Cu) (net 33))
 (segment (start 117.729 81.153) (end 118.237 80.645) (width 0.25) (layer F.Cu) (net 33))
 (via (at 117.729 81.153) (size 0.6) (drill 0.4) (layers F.Cu B.Cu) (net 33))
 (segment (start 113.919 81.153) (end 117.729 81.153) (width 0.25) (layer B.Cu) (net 33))
 (segment (start 113.792 81.28) (end 113.919 81.153) (width 0.25) (layer B.Cu) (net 33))
 (via (at 113.792 81.28) (size 0.6) (drill 0.4) (layers F.Cu B.Cu) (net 33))
 (segment (start 112.776 82.296) (end 113.792 81.28) (width 0.25) (layer F.Cu) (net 33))
 (segment (start 176.53 72.35) (end 189.23 72.35) (width 0.254) (layer B.Cu) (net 34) (status 800000))
 (segment (start 177.165 72.35) (end 176.53 72.35) (width 0.25) (layer B.Cu) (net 34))
 (segment (start 176.53 72.35) (end 171.918 72.35) (width 0.25) (layer B.Cu) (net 34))
 (segment (start 117.856 70.612) (end 115.697 72.771) (width 0.25) (layer F.Cu) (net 34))
 (via (at 117.856 70.612) (size 0.6) (drill 0.4) (layers F.Cu B.Cu) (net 34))
 (segment (start 170.18 70.612) (end 117.856 70.612) (width 0.25) (layer B.Cu) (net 34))
 (segment (start 171.918 72.35) (end 170.18 70.612) (width 0.25) (layer B.Cu) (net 34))
 (segment (start 115.697 72.771) (end 115.57 72.771) (width 0.25) (layer F.Cu) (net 34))
 (segment (start 115.57 63.246) (end 115.57 60.071) (width 0.25) (layer F.Cu) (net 34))
 (segment (start 115.57 66.421) (end 115.57 63.246) (width 0.25) (layer F.Cu) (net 34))
 (segment (start 115.57 69.596) (end 115.57 66.421) (width 0.25) (layer F.Cu) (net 34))
 (segment (start 115.57 72.771) (end 115.57 69.596) (width 0.25) (layer F.Cu) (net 34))
 (segment (start 115.57 75.946) (end 115.57 72.771) (width 0.25) (layer F.Cu) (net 34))
 (segment (start 115.57 79.121) (end 115.57 75.946) (width 0.25) (layer F.Cu) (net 34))
 (segment (start 115.57 82.296) (end 115.57 79.121) (width 0.25) (layer F.Cu) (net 34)))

